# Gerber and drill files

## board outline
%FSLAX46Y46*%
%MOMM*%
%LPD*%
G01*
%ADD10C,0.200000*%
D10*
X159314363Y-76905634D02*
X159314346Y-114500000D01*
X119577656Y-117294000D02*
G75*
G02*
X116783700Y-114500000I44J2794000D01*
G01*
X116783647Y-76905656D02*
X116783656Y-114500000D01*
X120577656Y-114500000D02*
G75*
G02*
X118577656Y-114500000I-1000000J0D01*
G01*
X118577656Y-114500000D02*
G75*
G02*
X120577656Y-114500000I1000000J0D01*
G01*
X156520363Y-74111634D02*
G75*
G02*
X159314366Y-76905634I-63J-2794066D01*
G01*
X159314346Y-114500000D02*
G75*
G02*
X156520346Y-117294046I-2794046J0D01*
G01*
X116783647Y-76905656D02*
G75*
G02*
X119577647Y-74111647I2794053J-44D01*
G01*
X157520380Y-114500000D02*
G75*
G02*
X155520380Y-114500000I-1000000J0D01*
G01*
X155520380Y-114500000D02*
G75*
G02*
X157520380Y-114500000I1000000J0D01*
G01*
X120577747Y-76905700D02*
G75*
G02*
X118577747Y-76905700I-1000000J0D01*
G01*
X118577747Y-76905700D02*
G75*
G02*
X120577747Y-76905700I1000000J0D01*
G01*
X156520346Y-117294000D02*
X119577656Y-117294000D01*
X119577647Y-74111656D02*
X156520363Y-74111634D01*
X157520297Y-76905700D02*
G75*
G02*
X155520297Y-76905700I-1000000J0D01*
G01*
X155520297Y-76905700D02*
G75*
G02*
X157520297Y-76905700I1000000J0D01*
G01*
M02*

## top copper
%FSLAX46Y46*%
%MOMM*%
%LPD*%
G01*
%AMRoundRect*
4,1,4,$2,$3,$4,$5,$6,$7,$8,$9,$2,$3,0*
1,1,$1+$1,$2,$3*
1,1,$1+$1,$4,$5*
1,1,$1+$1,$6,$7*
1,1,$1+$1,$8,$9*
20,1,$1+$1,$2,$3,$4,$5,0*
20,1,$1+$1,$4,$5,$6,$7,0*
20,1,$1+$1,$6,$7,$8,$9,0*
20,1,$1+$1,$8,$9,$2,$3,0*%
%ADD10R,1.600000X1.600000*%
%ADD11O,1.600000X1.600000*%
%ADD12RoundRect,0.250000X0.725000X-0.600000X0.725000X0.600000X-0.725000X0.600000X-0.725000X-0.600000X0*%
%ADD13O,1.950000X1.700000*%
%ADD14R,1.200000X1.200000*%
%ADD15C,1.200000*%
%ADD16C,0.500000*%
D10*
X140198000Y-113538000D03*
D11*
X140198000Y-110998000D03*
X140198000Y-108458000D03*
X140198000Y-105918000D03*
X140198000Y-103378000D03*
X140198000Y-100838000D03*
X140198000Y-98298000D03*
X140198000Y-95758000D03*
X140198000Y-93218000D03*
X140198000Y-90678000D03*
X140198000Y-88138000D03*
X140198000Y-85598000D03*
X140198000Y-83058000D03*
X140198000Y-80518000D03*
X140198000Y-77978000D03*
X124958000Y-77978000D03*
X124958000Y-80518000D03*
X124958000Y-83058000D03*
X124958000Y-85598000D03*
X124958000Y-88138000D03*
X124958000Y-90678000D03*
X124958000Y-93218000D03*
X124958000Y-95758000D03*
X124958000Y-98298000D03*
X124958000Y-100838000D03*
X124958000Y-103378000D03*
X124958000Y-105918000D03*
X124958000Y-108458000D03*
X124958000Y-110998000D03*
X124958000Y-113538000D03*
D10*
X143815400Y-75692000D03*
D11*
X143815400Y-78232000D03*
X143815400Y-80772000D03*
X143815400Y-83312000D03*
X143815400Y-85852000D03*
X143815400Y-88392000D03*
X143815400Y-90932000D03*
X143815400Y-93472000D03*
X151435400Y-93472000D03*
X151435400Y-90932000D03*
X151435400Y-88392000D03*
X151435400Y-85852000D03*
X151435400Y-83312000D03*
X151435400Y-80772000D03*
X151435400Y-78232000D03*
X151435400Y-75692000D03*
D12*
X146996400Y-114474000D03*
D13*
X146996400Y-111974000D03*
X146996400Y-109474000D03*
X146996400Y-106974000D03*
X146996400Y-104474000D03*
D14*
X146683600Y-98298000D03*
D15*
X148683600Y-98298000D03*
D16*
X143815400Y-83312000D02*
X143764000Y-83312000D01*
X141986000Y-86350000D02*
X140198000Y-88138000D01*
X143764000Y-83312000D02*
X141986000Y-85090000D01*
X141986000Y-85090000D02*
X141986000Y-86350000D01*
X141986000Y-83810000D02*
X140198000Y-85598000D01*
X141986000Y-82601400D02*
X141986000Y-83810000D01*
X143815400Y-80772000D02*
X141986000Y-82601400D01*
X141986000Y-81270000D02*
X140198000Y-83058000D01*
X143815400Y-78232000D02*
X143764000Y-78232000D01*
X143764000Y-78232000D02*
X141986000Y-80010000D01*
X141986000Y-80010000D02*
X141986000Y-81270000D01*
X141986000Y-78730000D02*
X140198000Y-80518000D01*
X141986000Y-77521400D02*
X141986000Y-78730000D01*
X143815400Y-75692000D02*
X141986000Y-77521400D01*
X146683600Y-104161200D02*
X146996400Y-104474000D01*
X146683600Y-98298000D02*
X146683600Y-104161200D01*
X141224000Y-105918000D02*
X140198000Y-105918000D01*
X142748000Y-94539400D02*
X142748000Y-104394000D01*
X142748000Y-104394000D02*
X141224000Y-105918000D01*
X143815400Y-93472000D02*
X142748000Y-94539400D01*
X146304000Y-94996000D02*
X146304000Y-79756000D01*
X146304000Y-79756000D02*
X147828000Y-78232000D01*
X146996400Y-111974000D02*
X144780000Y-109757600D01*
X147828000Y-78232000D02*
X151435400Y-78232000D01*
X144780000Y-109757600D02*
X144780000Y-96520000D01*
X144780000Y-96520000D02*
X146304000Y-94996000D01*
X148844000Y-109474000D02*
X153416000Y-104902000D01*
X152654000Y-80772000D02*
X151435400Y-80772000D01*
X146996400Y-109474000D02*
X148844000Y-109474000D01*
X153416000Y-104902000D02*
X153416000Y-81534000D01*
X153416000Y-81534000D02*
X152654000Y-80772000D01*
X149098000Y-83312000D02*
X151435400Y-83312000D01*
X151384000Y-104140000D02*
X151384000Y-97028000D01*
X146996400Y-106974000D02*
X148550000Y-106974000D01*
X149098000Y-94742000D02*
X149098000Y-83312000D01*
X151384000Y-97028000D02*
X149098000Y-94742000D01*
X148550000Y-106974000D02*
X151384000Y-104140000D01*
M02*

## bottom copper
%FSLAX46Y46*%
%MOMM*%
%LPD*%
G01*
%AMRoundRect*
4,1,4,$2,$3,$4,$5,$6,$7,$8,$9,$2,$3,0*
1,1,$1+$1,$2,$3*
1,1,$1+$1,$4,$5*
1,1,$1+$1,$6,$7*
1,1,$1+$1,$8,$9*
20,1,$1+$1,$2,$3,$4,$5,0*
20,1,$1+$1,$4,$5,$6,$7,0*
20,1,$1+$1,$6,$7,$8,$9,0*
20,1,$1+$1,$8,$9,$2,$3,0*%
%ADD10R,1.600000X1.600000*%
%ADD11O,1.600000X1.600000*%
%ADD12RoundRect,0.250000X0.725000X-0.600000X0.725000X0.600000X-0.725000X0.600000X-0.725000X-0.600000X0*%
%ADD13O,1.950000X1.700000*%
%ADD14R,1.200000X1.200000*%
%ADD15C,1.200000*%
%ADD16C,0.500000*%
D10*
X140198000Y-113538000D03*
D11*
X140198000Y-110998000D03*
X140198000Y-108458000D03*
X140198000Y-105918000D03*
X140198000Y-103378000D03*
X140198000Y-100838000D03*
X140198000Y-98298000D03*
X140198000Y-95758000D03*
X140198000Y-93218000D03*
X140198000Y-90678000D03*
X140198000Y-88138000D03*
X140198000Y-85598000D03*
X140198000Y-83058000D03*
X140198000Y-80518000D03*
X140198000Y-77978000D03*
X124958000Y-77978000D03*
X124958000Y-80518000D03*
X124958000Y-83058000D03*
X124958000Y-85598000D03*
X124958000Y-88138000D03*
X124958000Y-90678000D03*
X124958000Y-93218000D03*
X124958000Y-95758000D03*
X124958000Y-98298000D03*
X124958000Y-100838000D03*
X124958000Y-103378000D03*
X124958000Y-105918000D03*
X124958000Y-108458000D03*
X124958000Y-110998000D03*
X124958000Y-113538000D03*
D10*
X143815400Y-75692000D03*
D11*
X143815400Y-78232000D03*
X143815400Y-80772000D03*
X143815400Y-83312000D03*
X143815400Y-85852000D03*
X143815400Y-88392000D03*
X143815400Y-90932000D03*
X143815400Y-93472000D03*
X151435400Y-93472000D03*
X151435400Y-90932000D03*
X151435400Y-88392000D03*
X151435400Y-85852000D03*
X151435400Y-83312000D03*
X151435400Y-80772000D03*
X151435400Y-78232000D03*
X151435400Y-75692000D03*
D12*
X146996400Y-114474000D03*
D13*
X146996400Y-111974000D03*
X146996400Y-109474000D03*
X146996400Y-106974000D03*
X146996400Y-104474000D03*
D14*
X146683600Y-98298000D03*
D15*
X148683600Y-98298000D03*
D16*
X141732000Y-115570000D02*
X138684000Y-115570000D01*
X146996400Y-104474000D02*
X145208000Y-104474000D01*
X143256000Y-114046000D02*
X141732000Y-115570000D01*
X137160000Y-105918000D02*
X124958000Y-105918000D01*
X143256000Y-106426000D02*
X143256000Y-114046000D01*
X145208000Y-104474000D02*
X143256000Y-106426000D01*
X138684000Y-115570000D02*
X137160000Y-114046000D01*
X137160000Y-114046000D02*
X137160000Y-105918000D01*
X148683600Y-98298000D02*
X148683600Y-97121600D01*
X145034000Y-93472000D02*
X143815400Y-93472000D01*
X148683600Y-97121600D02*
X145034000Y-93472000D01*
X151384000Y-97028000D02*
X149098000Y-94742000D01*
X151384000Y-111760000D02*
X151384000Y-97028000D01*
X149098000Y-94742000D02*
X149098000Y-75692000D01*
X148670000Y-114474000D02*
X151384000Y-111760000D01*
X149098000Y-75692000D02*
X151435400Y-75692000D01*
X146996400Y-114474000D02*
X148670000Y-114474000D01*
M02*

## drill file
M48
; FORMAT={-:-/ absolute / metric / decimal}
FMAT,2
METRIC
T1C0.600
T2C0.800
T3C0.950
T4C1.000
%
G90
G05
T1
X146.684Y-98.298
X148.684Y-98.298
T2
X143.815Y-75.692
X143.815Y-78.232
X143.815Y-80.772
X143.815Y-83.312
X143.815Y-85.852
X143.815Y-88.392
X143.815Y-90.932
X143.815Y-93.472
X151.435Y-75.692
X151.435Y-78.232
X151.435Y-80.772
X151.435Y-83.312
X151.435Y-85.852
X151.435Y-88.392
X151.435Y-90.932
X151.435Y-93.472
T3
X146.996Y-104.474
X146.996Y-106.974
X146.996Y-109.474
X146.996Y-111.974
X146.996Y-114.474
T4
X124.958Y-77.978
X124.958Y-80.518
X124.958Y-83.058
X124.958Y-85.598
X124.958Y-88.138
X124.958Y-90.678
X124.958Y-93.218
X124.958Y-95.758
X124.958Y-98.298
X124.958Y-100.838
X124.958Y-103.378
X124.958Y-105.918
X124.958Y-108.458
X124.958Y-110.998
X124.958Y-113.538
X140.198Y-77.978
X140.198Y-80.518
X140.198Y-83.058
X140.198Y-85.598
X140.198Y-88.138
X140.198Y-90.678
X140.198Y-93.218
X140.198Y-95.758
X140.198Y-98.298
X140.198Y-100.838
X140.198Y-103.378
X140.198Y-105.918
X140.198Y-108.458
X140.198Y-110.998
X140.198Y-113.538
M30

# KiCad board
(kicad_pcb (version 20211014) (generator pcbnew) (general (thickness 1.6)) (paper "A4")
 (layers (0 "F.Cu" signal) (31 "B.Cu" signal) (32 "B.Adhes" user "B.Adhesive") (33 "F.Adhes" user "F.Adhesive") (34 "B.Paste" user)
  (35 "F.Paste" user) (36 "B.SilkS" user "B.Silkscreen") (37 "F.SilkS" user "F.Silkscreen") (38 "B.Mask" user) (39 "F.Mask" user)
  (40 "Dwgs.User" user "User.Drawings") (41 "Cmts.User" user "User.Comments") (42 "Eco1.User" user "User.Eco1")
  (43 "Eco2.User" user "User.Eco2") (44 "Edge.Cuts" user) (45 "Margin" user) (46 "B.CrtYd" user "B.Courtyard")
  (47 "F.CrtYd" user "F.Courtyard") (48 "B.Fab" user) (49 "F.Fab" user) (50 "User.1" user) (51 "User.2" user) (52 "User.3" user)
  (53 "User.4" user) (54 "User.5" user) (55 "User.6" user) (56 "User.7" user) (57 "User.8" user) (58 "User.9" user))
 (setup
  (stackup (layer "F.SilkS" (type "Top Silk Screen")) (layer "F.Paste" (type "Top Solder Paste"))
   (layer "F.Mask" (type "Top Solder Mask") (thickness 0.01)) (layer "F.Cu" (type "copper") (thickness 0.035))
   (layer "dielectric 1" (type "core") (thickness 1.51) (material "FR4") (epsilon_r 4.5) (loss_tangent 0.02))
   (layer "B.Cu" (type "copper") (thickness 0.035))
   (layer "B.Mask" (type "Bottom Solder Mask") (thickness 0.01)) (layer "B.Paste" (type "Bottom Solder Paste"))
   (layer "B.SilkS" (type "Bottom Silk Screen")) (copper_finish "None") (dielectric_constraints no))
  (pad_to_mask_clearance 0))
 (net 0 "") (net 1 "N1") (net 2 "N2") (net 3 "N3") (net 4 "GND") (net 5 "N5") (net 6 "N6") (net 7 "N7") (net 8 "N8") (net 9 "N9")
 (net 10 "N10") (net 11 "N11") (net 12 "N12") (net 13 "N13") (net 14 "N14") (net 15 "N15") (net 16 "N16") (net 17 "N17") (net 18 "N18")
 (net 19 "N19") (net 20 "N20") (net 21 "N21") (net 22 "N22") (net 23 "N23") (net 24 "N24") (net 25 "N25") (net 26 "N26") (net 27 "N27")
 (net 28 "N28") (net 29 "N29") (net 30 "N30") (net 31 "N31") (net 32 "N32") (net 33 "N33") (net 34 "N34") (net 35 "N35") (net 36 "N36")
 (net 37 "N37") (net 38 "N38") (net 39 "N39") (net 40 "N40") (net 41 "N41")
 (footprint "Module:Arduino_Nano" (layer "F.Cu") (at 140.198 113.538 180)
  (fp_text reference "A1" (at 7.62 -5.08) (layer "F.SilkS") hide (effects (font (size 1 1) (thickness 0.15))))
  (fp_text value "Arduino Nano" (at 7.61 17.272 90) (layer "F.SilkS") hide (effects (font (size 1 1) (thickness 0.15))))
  (pad "1" thru_hole rect (at 0 0 180) (size 1.6 1.6) (drill 1) (layers *.Cu *.Mask) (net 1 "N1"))
  (pad "2" thru_hole oval (at 0 2.54 180) (size 1.6 1.6) (drill 1) (layers *.Cu *.Mask) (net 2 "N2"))
  (pad "3" thru_hole oval (at 0 5.08 180) (size 1.6 1.6) (drill 1) (layers *.Cu *.Mask) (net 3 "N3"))
  (pad "4" thru_hole oval (at 0 7.62 180) (size 1.6 1.6) (drill 1) (layers *.Cu *.Mask) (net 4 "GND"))
  (pad "5" thru_hole oval (at 0 10.16 180) (size 1.6 1.6) (drill 1) (layers *.Cu *.Mask) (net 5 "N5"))
  (pad "6" thru_hole oval (at 0 12.7 180) (size 1.6 1.6) (drill 1) (layers *.Cu *.Mask) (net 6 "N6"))
  (pad "7" thru_hole oval (at 0 15.24 180) (size 1.6 1.6) (drill 1) (layers *.Cu *.Mask) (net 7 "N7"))
  (pad "8" thru_hole oval (at 0 17.78 180) (size 1.6 1.6) (drill 1) (layers *.Cu *.Mask) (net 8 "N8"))
  (pad "9" thru_hole oval (at 0 20.32 180) (size 1.6 1.6) (drill 1) (layers *.Cu *.Mask) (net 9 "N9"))
  (pad "10" thru_hole oval (at 0 22.86 180) (size 1.6 1.6) (drill 1) (layers *.Cu *.Mask) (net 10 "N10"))
  (pad "11" thru_hole oval (at 0 25.4 180) (size 1.6 1.6) (drill 1) (layers *.Cu *.Mask) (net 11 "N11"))
  (pad "12" thru_hole oval (at 0 27.94 180) (size 1.6 1.6) (drill 1) (layers *.Cu *.Mask) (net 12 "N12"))
  (pad "13" thru_hole oval (at 0 30.48 180) (size 1.6 1.6) (drill 1) (layers *.Cu *.Mask) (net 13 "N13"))
  (pad "14" thru_hole oval (at 0 33.02 180) (size 1.6 1.6) (drill 1) (layers *.Cu *.Mask) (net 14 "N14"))
  (pad "15" thru_hole oval (at 0 35.56 180) (size 1.6 1.6) (drill 1) (layers *.Cu *.Mask) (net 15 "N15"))
  (pad "16" thru_hole oval (at 15.24 35.56 180) (size 1.6 1.6) (drill 1) (layers *.Cu *.Mask) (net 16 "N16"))
  (pad "17" thru_hole oval (at 15.24 33.02 180) (size 1.6 1.6) (drill 1) (layers *.Cu *.Mask) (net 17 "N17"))
  (pad "18" thru_hole oval (at 15.24 30.48 180) (size 1.6 1.6) (drill 1) (layers *.Cu *.Mask) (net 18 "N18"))
  (pad "19" thru_hole oval (at 15.24 27.94 180) (size 1.6 1.6) (drill 1) (layers *.Cu *.Mask) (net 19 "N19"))
  (pad "20" thru_hole oval (at 15.24 25.4 180) (size 1.6 1.6) (drill 1) (layers *.Cu *.Mask) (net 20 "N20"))
  (pad "21" thru_hole oval (at 15.24 22.86 180) (size 1.6 1.6) (drill 1) (layers *.Cu *.Mask) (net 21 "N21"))
  (pad "22" thru_hole oval (at 15.24 20.32 180) (size 1.6 1.6) (drill 1) (layers *.Cu *.Mask) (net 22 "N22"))
  (pad "23" thru_hole oval (at 15.24 17.78 180) (size 1.6 1.6) (drill 1) (layers *.Cu *.Mask) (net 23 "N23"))
  (pad "24" thru_hole oval (at 15.24 15.24 180) (size 1.6 1.6) (drill 1) (layers *.Cu *.Mask) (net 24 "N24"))
  (pad "25" thru_hole oval (at 15.24 12.7 180) (size 1.6 1.6) (drill 1) (layers *.Cu *.Mask) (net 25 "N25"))
  (pad "26" thru_hole oval (at 15.24 10.16 180) (size 1.6 1.6) (drill 1) (layers *.Cu *.Mask) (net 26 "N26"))
  (pad "27" thru_hole oval (at 15.24 7.62 180) (size 1.6 1.6) (drill 1) (layers *.Cu *.Mask) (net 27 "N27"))
  (pad "28" thru_hole oval (at 15.24 5.08 180) (size 1.6 1.6) (drill 1) (layers *.Cu *.Mask) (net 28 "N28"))
  (pad "29" thru_hole oval (at 15.24 2.54 180) (size 1.6 1.6) (drill 1) (layers *.Cu *.Mask) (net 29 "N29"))
  (pad "30" thru_hole oval (at 15.24 0 180) (size 1.6 1.6) (drill 1) (layers *.Cu *.Mask) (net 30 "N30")))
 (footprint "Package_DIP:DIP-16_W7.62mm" (layer "F.Cu") (at 143.8154 75.692)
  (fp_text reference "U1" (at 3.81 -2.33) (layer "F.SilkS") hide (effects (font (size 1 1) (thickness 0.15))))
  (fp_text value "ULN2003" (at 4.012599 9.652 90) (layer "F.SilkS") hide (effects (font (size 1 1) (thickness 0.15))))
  (pad "1" thru_hole rect (at 0 0) (size 1.6 1.6) (drill 0.8) (layers *.Cu *.Mask) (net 14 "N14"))
  (pad "2" thru_hole oval (at 0 2.54) (size 1.6 1.6) (drill 0.8) (layers *.Cu *.Mask) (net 13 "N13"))
  (pad "3" thru_hole oval (at 0 5.08) (size 1.6 1.6) (drill 0.8) (layers *.Cu *.Mask) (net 12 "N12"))
  (pad "4" thru_hole oval (at 0 7.62) (size 1.6 1.6) (drill 0.8) (layers *.Cu *.Mask) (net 11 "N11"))
  (pad "5" thru_hole oval (at 0 10.16) (size 1.6 1.6) (drill 0.8) (layers *.Cu *.Mask) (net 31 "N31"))
  (pad "6" thru_hole oval (at 0 12.7) (size 1.6 1.6) (drill 0.8) (layers *.Cu *.Mask) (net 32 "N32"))
  (pad "7" thru_hole oval (at 0 15.24) (size 1.6 1.6) (drill 0.8) (layers *.Cu *.Mask) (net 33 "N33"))
  (pad "8" thru_hole oval (at 0 17.78) (size 1.6 1.6) (drill 0.8) (layers *.Cu *.Mask) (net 4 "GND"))
  (pad "9" thru_hole oval (at 7.62 17.78) (size 1.6 1.6) (drill 0.8) (layers *.Cu *.Mask) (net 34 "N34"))
  (pad "10" thru_hole oval (at 7.62 15.24) (size 1.6 1.6) (drill 0.8) (layers *.Cu *.Mask) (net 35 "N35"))
  (pad "11" thru_hole oval (at 7.62 12.7) (size 1.6 1.6) (drill 0.8) (layers *.Cu *.Mask) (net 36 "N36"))
  (pad "12" thru_hole oval (at 7.62 10.16) (size 1.6 1.6) (drill 0.8) (layers *.Cu *.Mask) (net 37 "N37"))
  (pad "13" thru_hole oval (at 7.62 7.62) (size 1.6 1.6) (drill 0.8) (layers *.Cu *.Mask) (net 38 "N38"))
  (pad "14" thru_hole oval (at 7.62 5.08) (size 1.6 1.6) (drill 0.8) (layers *.Cu *.Mask) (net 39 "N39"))
  (pad "15" thru_hole oval (at 7.62 2.54) (size 1.6 1.6) (drill 0.8) (layers *.Cu *.Mask) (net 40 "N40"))
  (pad "16" thru_hole oval (at 7.62 0) (size 1.6 1.6) (drill 0.8) (layers *.Cu *.Mask) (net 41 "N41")))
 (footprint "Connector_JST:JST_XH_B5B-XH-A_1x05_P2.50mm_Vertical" (layer "F.Cu") (at 146.9964 114.474 90)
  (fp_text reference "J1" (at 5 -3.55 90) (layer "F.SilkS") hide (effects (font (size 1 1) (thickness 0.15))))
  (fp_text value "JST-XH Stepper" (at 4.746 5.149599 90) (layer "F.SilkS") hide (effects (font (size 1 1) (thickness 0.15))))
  (pad "1" thru_hole roundrect (at 0 0 90) (size 1.7 1.95) (drill 0.95) (layers *.Cu *.Mask) (roundrect_rratio 0.1470588235) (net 41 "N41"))
  (pad "2" thru_hole oval (at 2.5 0 90) (size 1.7 1.95) (drill 0.95) (layers *.Cu *.Mask) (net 40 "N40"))
  (pad "3" thru_hole oval (at 5 0 90) (size 1.7 1.95) (drill 0.95) (layers *.Cu *.Mask) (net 39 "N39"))
  (pad "4" thru_hole oval (at 7.5 0 90) (size 1.7 1.95) (drill 0.95) (layers *.Cu *.Mask) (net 38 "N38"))
  (pad "5" thru_hole oval (at 10 0 90) (size 1.7 1.95) (drill 0.95) (layers *.Cu *.Mask) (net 27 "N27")))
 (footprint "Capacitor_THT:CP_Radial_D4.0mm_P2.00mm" (layer "F.Cu") (at 146.6836 98.298)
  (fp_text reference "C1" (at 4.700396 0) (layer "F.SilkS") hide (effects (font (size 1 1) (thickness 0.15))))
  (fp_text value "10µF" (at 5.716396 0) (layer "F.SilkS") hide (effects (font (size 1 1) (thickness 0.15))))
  (pad "1" thru_hole rect (at 0 0) (size 1.2 1.2) (drill 0.6) (layers *.Cu *.Mask) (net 27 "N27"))
  (pad "2" thru_hole circle (at 2 0) (size 1.2 1.2) (drill 0.6) (layers *.Cu *.Mask) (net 4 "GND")))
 (gr_line (start 159.314363 76.905634) (end 159.314346 114.5) (layer "Edge.Cuts") (width 0.2))
 (gr_arc (start 119.577656 117.294) (mid 117.602 116.475656) (end 116.783656 114.5) (layer "Edge.Cuts") (width 0.2))
 (gr_line (start 116.783647 76.905656) (end 116.783656 114.5) (layer "Edge.Cuts") (width 0.2))
 (gr_circle (center 119.577656 114.5) (end 120.577656 114.5) (layer "Edge.Cuts") (width 0.2) (fill none))
 (gr_arc (start 156.520363 74.111634) (mid 158.496 74.929997) (end 159.314363 76.905634) (layer "Edge.Cuts") (width 0.2))
 (gr_arc (start 159.314346 114.5) (mid 158.496 116.475644) (end 156.520346 117.294) (layer "Edge.Cuts") (width 0.2))
 (gr_arc (start 116.783647 76.905656) (mid 117.602 74.929993) (end 119.577647 74.111656) (layer "Edge.Cuts") (width 0.2))
 (gr_circle (center 156.52038 114.5) (end 157.52038 114.5) (layer "Edge.Cuts") (width 0.2) (fill none))
 (gr_circle (center 119.577747 76.9057) (end 120.577747 76.9057) (layer "Edge.Cuts") (width 0.2) (fill none))
 (gr_line (start 156.520346 117.294) (end 119.577656 117.294) (layer "Edge.Cuts") (width 0.2))
 (gr_line (start 119.577647 74.111656) (end 156.520363 74.111634) (layer "Edge.Cuts") (width 0.2))
 (gr_circle (center 156.520297 76.9057) (end 157.520297 76.9057) (layer "Edge.Cuts") (width 0.2) (fill none))
 (segment (start 143.8154 83.312) (end 143.764 83.312) (width 0.5) (layer "F.Cu") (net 11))
 (segment (start 141.986 86.35) (end 140.198 88.138) (width 0.5) (layer "F.Cu") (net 11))
 (segment (start 143.764 83.312) (end 141.986 85.09) (width 0.5) (layer "F.Cu") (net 11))
 (segment (start 141.986 85.09) (end 141.986 86.35) (width 0.5) (layer "F.Cu") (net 11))
 (segment (start 141.986 83.81) (end 140.198 85.598) (width 0.5) (layer "F.Cu") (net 12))
 (segment (start 141.986 82.6014) (end 141.986 83.81) (width 0.5) (layer "F.Cu") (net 12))
 (segment (start 143.8154 80.772) (end 141.986 82.6014) (width 0.5) (layer "F.Cu") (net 12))
 (segment (start 141.986 81.27) (end 140.198 83.058) (width 0.5) (layer "F.Cu") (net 13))
 (segment (start 143.8154 78.232) (end 143.764 78.232) (width 0.5) (layer "F.Cu") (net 13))
 (segment (start 143.764 78.232) (end 141.986 80.01) (width 0.5) (layer "F.Cu") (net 13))
 (segment (start 141.986 80.01) (end 141.986 81.27) (width 0.5) (layer "F.Cu") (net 13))
 (segment (start 141.986 78.73) (end 140.198 80.518) (width 0.5) (layer "F.Cu") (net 14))
 (segment (start 141.986 77.5214) (end 141.986 78.73) (width 0.5) (layer "F.Cu") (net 14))
 (segment (start 143.8154 75.692) (end 141.986 77.5214) (width 0.5) (layer "F.Cu") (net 14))
 (segment (start 146.6836 104.1612) (end 146.9964 104.474) (width 0.5) (layer "F.Cu") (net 27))
 (segment (start 146.6836 98.298) (end 146.6836 104.1612) (width 0.5) (layer "F.Cu") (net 27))
 (segment (start 141.732 115.57) (end 138.684 115.57) (width 0.5) (layer "B.Cu") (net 27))
 (segment (start 146.9964 104.474) (end 145.208 104.474) (width 0.5) (layer "B.Cu") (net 27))
 (segment (start 143.256 114.046) (end 141.732 115.57) (width 0.5) (layer "B.Cu") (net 27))
 (segment (start 137.16 105.918) (end 124.958 105.918) (width 0.5) (layer "B.Cu") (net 27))
 (segment (start 143.256 106.426) (end 143.256 114.046) (width 0.5) (layer "B.Cu") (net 27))
 (segment (start 145.208 104.474) (end 143.256 106.426) (width 0.5) (layer "B.Cu") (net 27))
 (segment (start 138.684 115.57) (end 137.16 114.046) (width 0.5) (layer "B.Cu") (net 27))
 (segment (start 137.16 114.046) (end 137.16 105.918) (width 0.5) (layer "B.Cu") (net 27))
 (segment (start 141.224 105.918) (end 140.198 105.918) (width 0.5) (layer "F.Cu") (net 4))
 (segment (start 142.748 94.5394) (end 142.748 104.394) (width 0.5) (layer "F.Cu") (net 4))
 (segment (start 142.748 104.394) (end 141.224 105.918) (width 0.5) (layer "F.Cu") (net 4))
 (segment (start 143.8154 93.472) (end 142.748 94.5394) (width 0.5) (layer "F.Cu") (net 4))
 (segment (start 148.6836 98.298) (end 148.6836 97.1216) (width 0.5) (layer "B.Cu") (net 4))
 (segment (start 145.034 93.472) (end 143.8154 93.472) (width 0.5) (layer "B.Cu") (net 4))
 (segment (start 148.6836 97.1216) (end 145.034 93.472) (width 0.5) (layer "B.Cu") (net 4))
 (segment (start 151.384 97.028) (end 149.098 94.742) (width 0.5) (layer "B.Cu") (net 41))
 (segment (start 151.384 111.76) (end 151.384 97.028) (width 0.5) (layer "B.Cu") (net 41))
 (segment (start 149.098 94.742) (end 149.098 75.692) (width 0.5) (layer "B.Cu") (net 41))
 (segment (start 148.67 114.474) (end 151.384 111.76) (width 0.5) (layer "B.Cu") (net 41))
 (segment (start 149.098 75.692) (end 151.4354 75.692) (width 0.5) (layer "B.Cu") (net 41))
 (segment (start 146.9964 114.474) (end 148.67 114.474) (width 0.5) (layer "B.Cu") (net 41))
 (segment (start 146.304 94.996) (end 146.304 79.756) (width 0.5) (layer "F.Cu") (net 40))
 (segment (start 146.304 79.756) (end 147.828 78.232) (width 0.5) (layer "F.Cu") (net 40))
 (segment (start 146.9964 111.974) (end 144.78 109.7576) (width 0.5) (layer "F.Cu") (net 40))
 (segment (start 147.828 78.232) (end 151.4354 78.232) (width 0.5) (layer "F.Cu") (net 40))
 (segment (start 144.78 109.7576) (end 144.78 96.52) (width 0.5) (layer "F.Cu") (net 40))
 (segment (start 144.78 96.52) (end 146.304 94.996) (width 0.5) (layer "F.Cu") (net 40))
 (segment (start 148.844 109.474) (end 153.416 104.902) (width 0.5) (layer "F.Cu") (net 39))
 (segment (start 152.654 80.772) (end 151.4354 80.772) (width 0.5) (layer "F.Cu") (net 39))
 (segment (start 146.9964 109.474) (end 148.844 109.474) (width 0.5) (layer "F.Cu") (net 39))
 (segment (start 153.416 104.902) (end 153.416 81.534) (width 0.5) (layer "F.Cu") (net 39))
 (segment (start 153.416 81.534) (end 152.654 80.772) (width 0.5) (layer "F.Cu") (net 39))
 (segment (start 149.098 83.312) (end 151.4354 83.312) (width 0.5) (layer "F.Cu") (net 38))
 (segment (start 151.384 104.14) (end 151.384 97.028) (width 0.5) (layer "F.Cu") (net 38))
 (segment (start 146.9964 106.974) (end 148.55 106.974) (width 0.5) (layer "F.Cu") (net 38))
 (segment (start 149.098 94.742) (end 149.098 83.312) (width 0.5) (layer "F.Cu") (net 38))
 (segment (start 151.384 97.028) (end 149.098 94.742) (width 0.5) (layer "F.Cu") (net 38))
 (segment (start 148.55 106.974) (end 151.384 104.14) (width 0.5) (layer "F.Cu") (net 38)))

